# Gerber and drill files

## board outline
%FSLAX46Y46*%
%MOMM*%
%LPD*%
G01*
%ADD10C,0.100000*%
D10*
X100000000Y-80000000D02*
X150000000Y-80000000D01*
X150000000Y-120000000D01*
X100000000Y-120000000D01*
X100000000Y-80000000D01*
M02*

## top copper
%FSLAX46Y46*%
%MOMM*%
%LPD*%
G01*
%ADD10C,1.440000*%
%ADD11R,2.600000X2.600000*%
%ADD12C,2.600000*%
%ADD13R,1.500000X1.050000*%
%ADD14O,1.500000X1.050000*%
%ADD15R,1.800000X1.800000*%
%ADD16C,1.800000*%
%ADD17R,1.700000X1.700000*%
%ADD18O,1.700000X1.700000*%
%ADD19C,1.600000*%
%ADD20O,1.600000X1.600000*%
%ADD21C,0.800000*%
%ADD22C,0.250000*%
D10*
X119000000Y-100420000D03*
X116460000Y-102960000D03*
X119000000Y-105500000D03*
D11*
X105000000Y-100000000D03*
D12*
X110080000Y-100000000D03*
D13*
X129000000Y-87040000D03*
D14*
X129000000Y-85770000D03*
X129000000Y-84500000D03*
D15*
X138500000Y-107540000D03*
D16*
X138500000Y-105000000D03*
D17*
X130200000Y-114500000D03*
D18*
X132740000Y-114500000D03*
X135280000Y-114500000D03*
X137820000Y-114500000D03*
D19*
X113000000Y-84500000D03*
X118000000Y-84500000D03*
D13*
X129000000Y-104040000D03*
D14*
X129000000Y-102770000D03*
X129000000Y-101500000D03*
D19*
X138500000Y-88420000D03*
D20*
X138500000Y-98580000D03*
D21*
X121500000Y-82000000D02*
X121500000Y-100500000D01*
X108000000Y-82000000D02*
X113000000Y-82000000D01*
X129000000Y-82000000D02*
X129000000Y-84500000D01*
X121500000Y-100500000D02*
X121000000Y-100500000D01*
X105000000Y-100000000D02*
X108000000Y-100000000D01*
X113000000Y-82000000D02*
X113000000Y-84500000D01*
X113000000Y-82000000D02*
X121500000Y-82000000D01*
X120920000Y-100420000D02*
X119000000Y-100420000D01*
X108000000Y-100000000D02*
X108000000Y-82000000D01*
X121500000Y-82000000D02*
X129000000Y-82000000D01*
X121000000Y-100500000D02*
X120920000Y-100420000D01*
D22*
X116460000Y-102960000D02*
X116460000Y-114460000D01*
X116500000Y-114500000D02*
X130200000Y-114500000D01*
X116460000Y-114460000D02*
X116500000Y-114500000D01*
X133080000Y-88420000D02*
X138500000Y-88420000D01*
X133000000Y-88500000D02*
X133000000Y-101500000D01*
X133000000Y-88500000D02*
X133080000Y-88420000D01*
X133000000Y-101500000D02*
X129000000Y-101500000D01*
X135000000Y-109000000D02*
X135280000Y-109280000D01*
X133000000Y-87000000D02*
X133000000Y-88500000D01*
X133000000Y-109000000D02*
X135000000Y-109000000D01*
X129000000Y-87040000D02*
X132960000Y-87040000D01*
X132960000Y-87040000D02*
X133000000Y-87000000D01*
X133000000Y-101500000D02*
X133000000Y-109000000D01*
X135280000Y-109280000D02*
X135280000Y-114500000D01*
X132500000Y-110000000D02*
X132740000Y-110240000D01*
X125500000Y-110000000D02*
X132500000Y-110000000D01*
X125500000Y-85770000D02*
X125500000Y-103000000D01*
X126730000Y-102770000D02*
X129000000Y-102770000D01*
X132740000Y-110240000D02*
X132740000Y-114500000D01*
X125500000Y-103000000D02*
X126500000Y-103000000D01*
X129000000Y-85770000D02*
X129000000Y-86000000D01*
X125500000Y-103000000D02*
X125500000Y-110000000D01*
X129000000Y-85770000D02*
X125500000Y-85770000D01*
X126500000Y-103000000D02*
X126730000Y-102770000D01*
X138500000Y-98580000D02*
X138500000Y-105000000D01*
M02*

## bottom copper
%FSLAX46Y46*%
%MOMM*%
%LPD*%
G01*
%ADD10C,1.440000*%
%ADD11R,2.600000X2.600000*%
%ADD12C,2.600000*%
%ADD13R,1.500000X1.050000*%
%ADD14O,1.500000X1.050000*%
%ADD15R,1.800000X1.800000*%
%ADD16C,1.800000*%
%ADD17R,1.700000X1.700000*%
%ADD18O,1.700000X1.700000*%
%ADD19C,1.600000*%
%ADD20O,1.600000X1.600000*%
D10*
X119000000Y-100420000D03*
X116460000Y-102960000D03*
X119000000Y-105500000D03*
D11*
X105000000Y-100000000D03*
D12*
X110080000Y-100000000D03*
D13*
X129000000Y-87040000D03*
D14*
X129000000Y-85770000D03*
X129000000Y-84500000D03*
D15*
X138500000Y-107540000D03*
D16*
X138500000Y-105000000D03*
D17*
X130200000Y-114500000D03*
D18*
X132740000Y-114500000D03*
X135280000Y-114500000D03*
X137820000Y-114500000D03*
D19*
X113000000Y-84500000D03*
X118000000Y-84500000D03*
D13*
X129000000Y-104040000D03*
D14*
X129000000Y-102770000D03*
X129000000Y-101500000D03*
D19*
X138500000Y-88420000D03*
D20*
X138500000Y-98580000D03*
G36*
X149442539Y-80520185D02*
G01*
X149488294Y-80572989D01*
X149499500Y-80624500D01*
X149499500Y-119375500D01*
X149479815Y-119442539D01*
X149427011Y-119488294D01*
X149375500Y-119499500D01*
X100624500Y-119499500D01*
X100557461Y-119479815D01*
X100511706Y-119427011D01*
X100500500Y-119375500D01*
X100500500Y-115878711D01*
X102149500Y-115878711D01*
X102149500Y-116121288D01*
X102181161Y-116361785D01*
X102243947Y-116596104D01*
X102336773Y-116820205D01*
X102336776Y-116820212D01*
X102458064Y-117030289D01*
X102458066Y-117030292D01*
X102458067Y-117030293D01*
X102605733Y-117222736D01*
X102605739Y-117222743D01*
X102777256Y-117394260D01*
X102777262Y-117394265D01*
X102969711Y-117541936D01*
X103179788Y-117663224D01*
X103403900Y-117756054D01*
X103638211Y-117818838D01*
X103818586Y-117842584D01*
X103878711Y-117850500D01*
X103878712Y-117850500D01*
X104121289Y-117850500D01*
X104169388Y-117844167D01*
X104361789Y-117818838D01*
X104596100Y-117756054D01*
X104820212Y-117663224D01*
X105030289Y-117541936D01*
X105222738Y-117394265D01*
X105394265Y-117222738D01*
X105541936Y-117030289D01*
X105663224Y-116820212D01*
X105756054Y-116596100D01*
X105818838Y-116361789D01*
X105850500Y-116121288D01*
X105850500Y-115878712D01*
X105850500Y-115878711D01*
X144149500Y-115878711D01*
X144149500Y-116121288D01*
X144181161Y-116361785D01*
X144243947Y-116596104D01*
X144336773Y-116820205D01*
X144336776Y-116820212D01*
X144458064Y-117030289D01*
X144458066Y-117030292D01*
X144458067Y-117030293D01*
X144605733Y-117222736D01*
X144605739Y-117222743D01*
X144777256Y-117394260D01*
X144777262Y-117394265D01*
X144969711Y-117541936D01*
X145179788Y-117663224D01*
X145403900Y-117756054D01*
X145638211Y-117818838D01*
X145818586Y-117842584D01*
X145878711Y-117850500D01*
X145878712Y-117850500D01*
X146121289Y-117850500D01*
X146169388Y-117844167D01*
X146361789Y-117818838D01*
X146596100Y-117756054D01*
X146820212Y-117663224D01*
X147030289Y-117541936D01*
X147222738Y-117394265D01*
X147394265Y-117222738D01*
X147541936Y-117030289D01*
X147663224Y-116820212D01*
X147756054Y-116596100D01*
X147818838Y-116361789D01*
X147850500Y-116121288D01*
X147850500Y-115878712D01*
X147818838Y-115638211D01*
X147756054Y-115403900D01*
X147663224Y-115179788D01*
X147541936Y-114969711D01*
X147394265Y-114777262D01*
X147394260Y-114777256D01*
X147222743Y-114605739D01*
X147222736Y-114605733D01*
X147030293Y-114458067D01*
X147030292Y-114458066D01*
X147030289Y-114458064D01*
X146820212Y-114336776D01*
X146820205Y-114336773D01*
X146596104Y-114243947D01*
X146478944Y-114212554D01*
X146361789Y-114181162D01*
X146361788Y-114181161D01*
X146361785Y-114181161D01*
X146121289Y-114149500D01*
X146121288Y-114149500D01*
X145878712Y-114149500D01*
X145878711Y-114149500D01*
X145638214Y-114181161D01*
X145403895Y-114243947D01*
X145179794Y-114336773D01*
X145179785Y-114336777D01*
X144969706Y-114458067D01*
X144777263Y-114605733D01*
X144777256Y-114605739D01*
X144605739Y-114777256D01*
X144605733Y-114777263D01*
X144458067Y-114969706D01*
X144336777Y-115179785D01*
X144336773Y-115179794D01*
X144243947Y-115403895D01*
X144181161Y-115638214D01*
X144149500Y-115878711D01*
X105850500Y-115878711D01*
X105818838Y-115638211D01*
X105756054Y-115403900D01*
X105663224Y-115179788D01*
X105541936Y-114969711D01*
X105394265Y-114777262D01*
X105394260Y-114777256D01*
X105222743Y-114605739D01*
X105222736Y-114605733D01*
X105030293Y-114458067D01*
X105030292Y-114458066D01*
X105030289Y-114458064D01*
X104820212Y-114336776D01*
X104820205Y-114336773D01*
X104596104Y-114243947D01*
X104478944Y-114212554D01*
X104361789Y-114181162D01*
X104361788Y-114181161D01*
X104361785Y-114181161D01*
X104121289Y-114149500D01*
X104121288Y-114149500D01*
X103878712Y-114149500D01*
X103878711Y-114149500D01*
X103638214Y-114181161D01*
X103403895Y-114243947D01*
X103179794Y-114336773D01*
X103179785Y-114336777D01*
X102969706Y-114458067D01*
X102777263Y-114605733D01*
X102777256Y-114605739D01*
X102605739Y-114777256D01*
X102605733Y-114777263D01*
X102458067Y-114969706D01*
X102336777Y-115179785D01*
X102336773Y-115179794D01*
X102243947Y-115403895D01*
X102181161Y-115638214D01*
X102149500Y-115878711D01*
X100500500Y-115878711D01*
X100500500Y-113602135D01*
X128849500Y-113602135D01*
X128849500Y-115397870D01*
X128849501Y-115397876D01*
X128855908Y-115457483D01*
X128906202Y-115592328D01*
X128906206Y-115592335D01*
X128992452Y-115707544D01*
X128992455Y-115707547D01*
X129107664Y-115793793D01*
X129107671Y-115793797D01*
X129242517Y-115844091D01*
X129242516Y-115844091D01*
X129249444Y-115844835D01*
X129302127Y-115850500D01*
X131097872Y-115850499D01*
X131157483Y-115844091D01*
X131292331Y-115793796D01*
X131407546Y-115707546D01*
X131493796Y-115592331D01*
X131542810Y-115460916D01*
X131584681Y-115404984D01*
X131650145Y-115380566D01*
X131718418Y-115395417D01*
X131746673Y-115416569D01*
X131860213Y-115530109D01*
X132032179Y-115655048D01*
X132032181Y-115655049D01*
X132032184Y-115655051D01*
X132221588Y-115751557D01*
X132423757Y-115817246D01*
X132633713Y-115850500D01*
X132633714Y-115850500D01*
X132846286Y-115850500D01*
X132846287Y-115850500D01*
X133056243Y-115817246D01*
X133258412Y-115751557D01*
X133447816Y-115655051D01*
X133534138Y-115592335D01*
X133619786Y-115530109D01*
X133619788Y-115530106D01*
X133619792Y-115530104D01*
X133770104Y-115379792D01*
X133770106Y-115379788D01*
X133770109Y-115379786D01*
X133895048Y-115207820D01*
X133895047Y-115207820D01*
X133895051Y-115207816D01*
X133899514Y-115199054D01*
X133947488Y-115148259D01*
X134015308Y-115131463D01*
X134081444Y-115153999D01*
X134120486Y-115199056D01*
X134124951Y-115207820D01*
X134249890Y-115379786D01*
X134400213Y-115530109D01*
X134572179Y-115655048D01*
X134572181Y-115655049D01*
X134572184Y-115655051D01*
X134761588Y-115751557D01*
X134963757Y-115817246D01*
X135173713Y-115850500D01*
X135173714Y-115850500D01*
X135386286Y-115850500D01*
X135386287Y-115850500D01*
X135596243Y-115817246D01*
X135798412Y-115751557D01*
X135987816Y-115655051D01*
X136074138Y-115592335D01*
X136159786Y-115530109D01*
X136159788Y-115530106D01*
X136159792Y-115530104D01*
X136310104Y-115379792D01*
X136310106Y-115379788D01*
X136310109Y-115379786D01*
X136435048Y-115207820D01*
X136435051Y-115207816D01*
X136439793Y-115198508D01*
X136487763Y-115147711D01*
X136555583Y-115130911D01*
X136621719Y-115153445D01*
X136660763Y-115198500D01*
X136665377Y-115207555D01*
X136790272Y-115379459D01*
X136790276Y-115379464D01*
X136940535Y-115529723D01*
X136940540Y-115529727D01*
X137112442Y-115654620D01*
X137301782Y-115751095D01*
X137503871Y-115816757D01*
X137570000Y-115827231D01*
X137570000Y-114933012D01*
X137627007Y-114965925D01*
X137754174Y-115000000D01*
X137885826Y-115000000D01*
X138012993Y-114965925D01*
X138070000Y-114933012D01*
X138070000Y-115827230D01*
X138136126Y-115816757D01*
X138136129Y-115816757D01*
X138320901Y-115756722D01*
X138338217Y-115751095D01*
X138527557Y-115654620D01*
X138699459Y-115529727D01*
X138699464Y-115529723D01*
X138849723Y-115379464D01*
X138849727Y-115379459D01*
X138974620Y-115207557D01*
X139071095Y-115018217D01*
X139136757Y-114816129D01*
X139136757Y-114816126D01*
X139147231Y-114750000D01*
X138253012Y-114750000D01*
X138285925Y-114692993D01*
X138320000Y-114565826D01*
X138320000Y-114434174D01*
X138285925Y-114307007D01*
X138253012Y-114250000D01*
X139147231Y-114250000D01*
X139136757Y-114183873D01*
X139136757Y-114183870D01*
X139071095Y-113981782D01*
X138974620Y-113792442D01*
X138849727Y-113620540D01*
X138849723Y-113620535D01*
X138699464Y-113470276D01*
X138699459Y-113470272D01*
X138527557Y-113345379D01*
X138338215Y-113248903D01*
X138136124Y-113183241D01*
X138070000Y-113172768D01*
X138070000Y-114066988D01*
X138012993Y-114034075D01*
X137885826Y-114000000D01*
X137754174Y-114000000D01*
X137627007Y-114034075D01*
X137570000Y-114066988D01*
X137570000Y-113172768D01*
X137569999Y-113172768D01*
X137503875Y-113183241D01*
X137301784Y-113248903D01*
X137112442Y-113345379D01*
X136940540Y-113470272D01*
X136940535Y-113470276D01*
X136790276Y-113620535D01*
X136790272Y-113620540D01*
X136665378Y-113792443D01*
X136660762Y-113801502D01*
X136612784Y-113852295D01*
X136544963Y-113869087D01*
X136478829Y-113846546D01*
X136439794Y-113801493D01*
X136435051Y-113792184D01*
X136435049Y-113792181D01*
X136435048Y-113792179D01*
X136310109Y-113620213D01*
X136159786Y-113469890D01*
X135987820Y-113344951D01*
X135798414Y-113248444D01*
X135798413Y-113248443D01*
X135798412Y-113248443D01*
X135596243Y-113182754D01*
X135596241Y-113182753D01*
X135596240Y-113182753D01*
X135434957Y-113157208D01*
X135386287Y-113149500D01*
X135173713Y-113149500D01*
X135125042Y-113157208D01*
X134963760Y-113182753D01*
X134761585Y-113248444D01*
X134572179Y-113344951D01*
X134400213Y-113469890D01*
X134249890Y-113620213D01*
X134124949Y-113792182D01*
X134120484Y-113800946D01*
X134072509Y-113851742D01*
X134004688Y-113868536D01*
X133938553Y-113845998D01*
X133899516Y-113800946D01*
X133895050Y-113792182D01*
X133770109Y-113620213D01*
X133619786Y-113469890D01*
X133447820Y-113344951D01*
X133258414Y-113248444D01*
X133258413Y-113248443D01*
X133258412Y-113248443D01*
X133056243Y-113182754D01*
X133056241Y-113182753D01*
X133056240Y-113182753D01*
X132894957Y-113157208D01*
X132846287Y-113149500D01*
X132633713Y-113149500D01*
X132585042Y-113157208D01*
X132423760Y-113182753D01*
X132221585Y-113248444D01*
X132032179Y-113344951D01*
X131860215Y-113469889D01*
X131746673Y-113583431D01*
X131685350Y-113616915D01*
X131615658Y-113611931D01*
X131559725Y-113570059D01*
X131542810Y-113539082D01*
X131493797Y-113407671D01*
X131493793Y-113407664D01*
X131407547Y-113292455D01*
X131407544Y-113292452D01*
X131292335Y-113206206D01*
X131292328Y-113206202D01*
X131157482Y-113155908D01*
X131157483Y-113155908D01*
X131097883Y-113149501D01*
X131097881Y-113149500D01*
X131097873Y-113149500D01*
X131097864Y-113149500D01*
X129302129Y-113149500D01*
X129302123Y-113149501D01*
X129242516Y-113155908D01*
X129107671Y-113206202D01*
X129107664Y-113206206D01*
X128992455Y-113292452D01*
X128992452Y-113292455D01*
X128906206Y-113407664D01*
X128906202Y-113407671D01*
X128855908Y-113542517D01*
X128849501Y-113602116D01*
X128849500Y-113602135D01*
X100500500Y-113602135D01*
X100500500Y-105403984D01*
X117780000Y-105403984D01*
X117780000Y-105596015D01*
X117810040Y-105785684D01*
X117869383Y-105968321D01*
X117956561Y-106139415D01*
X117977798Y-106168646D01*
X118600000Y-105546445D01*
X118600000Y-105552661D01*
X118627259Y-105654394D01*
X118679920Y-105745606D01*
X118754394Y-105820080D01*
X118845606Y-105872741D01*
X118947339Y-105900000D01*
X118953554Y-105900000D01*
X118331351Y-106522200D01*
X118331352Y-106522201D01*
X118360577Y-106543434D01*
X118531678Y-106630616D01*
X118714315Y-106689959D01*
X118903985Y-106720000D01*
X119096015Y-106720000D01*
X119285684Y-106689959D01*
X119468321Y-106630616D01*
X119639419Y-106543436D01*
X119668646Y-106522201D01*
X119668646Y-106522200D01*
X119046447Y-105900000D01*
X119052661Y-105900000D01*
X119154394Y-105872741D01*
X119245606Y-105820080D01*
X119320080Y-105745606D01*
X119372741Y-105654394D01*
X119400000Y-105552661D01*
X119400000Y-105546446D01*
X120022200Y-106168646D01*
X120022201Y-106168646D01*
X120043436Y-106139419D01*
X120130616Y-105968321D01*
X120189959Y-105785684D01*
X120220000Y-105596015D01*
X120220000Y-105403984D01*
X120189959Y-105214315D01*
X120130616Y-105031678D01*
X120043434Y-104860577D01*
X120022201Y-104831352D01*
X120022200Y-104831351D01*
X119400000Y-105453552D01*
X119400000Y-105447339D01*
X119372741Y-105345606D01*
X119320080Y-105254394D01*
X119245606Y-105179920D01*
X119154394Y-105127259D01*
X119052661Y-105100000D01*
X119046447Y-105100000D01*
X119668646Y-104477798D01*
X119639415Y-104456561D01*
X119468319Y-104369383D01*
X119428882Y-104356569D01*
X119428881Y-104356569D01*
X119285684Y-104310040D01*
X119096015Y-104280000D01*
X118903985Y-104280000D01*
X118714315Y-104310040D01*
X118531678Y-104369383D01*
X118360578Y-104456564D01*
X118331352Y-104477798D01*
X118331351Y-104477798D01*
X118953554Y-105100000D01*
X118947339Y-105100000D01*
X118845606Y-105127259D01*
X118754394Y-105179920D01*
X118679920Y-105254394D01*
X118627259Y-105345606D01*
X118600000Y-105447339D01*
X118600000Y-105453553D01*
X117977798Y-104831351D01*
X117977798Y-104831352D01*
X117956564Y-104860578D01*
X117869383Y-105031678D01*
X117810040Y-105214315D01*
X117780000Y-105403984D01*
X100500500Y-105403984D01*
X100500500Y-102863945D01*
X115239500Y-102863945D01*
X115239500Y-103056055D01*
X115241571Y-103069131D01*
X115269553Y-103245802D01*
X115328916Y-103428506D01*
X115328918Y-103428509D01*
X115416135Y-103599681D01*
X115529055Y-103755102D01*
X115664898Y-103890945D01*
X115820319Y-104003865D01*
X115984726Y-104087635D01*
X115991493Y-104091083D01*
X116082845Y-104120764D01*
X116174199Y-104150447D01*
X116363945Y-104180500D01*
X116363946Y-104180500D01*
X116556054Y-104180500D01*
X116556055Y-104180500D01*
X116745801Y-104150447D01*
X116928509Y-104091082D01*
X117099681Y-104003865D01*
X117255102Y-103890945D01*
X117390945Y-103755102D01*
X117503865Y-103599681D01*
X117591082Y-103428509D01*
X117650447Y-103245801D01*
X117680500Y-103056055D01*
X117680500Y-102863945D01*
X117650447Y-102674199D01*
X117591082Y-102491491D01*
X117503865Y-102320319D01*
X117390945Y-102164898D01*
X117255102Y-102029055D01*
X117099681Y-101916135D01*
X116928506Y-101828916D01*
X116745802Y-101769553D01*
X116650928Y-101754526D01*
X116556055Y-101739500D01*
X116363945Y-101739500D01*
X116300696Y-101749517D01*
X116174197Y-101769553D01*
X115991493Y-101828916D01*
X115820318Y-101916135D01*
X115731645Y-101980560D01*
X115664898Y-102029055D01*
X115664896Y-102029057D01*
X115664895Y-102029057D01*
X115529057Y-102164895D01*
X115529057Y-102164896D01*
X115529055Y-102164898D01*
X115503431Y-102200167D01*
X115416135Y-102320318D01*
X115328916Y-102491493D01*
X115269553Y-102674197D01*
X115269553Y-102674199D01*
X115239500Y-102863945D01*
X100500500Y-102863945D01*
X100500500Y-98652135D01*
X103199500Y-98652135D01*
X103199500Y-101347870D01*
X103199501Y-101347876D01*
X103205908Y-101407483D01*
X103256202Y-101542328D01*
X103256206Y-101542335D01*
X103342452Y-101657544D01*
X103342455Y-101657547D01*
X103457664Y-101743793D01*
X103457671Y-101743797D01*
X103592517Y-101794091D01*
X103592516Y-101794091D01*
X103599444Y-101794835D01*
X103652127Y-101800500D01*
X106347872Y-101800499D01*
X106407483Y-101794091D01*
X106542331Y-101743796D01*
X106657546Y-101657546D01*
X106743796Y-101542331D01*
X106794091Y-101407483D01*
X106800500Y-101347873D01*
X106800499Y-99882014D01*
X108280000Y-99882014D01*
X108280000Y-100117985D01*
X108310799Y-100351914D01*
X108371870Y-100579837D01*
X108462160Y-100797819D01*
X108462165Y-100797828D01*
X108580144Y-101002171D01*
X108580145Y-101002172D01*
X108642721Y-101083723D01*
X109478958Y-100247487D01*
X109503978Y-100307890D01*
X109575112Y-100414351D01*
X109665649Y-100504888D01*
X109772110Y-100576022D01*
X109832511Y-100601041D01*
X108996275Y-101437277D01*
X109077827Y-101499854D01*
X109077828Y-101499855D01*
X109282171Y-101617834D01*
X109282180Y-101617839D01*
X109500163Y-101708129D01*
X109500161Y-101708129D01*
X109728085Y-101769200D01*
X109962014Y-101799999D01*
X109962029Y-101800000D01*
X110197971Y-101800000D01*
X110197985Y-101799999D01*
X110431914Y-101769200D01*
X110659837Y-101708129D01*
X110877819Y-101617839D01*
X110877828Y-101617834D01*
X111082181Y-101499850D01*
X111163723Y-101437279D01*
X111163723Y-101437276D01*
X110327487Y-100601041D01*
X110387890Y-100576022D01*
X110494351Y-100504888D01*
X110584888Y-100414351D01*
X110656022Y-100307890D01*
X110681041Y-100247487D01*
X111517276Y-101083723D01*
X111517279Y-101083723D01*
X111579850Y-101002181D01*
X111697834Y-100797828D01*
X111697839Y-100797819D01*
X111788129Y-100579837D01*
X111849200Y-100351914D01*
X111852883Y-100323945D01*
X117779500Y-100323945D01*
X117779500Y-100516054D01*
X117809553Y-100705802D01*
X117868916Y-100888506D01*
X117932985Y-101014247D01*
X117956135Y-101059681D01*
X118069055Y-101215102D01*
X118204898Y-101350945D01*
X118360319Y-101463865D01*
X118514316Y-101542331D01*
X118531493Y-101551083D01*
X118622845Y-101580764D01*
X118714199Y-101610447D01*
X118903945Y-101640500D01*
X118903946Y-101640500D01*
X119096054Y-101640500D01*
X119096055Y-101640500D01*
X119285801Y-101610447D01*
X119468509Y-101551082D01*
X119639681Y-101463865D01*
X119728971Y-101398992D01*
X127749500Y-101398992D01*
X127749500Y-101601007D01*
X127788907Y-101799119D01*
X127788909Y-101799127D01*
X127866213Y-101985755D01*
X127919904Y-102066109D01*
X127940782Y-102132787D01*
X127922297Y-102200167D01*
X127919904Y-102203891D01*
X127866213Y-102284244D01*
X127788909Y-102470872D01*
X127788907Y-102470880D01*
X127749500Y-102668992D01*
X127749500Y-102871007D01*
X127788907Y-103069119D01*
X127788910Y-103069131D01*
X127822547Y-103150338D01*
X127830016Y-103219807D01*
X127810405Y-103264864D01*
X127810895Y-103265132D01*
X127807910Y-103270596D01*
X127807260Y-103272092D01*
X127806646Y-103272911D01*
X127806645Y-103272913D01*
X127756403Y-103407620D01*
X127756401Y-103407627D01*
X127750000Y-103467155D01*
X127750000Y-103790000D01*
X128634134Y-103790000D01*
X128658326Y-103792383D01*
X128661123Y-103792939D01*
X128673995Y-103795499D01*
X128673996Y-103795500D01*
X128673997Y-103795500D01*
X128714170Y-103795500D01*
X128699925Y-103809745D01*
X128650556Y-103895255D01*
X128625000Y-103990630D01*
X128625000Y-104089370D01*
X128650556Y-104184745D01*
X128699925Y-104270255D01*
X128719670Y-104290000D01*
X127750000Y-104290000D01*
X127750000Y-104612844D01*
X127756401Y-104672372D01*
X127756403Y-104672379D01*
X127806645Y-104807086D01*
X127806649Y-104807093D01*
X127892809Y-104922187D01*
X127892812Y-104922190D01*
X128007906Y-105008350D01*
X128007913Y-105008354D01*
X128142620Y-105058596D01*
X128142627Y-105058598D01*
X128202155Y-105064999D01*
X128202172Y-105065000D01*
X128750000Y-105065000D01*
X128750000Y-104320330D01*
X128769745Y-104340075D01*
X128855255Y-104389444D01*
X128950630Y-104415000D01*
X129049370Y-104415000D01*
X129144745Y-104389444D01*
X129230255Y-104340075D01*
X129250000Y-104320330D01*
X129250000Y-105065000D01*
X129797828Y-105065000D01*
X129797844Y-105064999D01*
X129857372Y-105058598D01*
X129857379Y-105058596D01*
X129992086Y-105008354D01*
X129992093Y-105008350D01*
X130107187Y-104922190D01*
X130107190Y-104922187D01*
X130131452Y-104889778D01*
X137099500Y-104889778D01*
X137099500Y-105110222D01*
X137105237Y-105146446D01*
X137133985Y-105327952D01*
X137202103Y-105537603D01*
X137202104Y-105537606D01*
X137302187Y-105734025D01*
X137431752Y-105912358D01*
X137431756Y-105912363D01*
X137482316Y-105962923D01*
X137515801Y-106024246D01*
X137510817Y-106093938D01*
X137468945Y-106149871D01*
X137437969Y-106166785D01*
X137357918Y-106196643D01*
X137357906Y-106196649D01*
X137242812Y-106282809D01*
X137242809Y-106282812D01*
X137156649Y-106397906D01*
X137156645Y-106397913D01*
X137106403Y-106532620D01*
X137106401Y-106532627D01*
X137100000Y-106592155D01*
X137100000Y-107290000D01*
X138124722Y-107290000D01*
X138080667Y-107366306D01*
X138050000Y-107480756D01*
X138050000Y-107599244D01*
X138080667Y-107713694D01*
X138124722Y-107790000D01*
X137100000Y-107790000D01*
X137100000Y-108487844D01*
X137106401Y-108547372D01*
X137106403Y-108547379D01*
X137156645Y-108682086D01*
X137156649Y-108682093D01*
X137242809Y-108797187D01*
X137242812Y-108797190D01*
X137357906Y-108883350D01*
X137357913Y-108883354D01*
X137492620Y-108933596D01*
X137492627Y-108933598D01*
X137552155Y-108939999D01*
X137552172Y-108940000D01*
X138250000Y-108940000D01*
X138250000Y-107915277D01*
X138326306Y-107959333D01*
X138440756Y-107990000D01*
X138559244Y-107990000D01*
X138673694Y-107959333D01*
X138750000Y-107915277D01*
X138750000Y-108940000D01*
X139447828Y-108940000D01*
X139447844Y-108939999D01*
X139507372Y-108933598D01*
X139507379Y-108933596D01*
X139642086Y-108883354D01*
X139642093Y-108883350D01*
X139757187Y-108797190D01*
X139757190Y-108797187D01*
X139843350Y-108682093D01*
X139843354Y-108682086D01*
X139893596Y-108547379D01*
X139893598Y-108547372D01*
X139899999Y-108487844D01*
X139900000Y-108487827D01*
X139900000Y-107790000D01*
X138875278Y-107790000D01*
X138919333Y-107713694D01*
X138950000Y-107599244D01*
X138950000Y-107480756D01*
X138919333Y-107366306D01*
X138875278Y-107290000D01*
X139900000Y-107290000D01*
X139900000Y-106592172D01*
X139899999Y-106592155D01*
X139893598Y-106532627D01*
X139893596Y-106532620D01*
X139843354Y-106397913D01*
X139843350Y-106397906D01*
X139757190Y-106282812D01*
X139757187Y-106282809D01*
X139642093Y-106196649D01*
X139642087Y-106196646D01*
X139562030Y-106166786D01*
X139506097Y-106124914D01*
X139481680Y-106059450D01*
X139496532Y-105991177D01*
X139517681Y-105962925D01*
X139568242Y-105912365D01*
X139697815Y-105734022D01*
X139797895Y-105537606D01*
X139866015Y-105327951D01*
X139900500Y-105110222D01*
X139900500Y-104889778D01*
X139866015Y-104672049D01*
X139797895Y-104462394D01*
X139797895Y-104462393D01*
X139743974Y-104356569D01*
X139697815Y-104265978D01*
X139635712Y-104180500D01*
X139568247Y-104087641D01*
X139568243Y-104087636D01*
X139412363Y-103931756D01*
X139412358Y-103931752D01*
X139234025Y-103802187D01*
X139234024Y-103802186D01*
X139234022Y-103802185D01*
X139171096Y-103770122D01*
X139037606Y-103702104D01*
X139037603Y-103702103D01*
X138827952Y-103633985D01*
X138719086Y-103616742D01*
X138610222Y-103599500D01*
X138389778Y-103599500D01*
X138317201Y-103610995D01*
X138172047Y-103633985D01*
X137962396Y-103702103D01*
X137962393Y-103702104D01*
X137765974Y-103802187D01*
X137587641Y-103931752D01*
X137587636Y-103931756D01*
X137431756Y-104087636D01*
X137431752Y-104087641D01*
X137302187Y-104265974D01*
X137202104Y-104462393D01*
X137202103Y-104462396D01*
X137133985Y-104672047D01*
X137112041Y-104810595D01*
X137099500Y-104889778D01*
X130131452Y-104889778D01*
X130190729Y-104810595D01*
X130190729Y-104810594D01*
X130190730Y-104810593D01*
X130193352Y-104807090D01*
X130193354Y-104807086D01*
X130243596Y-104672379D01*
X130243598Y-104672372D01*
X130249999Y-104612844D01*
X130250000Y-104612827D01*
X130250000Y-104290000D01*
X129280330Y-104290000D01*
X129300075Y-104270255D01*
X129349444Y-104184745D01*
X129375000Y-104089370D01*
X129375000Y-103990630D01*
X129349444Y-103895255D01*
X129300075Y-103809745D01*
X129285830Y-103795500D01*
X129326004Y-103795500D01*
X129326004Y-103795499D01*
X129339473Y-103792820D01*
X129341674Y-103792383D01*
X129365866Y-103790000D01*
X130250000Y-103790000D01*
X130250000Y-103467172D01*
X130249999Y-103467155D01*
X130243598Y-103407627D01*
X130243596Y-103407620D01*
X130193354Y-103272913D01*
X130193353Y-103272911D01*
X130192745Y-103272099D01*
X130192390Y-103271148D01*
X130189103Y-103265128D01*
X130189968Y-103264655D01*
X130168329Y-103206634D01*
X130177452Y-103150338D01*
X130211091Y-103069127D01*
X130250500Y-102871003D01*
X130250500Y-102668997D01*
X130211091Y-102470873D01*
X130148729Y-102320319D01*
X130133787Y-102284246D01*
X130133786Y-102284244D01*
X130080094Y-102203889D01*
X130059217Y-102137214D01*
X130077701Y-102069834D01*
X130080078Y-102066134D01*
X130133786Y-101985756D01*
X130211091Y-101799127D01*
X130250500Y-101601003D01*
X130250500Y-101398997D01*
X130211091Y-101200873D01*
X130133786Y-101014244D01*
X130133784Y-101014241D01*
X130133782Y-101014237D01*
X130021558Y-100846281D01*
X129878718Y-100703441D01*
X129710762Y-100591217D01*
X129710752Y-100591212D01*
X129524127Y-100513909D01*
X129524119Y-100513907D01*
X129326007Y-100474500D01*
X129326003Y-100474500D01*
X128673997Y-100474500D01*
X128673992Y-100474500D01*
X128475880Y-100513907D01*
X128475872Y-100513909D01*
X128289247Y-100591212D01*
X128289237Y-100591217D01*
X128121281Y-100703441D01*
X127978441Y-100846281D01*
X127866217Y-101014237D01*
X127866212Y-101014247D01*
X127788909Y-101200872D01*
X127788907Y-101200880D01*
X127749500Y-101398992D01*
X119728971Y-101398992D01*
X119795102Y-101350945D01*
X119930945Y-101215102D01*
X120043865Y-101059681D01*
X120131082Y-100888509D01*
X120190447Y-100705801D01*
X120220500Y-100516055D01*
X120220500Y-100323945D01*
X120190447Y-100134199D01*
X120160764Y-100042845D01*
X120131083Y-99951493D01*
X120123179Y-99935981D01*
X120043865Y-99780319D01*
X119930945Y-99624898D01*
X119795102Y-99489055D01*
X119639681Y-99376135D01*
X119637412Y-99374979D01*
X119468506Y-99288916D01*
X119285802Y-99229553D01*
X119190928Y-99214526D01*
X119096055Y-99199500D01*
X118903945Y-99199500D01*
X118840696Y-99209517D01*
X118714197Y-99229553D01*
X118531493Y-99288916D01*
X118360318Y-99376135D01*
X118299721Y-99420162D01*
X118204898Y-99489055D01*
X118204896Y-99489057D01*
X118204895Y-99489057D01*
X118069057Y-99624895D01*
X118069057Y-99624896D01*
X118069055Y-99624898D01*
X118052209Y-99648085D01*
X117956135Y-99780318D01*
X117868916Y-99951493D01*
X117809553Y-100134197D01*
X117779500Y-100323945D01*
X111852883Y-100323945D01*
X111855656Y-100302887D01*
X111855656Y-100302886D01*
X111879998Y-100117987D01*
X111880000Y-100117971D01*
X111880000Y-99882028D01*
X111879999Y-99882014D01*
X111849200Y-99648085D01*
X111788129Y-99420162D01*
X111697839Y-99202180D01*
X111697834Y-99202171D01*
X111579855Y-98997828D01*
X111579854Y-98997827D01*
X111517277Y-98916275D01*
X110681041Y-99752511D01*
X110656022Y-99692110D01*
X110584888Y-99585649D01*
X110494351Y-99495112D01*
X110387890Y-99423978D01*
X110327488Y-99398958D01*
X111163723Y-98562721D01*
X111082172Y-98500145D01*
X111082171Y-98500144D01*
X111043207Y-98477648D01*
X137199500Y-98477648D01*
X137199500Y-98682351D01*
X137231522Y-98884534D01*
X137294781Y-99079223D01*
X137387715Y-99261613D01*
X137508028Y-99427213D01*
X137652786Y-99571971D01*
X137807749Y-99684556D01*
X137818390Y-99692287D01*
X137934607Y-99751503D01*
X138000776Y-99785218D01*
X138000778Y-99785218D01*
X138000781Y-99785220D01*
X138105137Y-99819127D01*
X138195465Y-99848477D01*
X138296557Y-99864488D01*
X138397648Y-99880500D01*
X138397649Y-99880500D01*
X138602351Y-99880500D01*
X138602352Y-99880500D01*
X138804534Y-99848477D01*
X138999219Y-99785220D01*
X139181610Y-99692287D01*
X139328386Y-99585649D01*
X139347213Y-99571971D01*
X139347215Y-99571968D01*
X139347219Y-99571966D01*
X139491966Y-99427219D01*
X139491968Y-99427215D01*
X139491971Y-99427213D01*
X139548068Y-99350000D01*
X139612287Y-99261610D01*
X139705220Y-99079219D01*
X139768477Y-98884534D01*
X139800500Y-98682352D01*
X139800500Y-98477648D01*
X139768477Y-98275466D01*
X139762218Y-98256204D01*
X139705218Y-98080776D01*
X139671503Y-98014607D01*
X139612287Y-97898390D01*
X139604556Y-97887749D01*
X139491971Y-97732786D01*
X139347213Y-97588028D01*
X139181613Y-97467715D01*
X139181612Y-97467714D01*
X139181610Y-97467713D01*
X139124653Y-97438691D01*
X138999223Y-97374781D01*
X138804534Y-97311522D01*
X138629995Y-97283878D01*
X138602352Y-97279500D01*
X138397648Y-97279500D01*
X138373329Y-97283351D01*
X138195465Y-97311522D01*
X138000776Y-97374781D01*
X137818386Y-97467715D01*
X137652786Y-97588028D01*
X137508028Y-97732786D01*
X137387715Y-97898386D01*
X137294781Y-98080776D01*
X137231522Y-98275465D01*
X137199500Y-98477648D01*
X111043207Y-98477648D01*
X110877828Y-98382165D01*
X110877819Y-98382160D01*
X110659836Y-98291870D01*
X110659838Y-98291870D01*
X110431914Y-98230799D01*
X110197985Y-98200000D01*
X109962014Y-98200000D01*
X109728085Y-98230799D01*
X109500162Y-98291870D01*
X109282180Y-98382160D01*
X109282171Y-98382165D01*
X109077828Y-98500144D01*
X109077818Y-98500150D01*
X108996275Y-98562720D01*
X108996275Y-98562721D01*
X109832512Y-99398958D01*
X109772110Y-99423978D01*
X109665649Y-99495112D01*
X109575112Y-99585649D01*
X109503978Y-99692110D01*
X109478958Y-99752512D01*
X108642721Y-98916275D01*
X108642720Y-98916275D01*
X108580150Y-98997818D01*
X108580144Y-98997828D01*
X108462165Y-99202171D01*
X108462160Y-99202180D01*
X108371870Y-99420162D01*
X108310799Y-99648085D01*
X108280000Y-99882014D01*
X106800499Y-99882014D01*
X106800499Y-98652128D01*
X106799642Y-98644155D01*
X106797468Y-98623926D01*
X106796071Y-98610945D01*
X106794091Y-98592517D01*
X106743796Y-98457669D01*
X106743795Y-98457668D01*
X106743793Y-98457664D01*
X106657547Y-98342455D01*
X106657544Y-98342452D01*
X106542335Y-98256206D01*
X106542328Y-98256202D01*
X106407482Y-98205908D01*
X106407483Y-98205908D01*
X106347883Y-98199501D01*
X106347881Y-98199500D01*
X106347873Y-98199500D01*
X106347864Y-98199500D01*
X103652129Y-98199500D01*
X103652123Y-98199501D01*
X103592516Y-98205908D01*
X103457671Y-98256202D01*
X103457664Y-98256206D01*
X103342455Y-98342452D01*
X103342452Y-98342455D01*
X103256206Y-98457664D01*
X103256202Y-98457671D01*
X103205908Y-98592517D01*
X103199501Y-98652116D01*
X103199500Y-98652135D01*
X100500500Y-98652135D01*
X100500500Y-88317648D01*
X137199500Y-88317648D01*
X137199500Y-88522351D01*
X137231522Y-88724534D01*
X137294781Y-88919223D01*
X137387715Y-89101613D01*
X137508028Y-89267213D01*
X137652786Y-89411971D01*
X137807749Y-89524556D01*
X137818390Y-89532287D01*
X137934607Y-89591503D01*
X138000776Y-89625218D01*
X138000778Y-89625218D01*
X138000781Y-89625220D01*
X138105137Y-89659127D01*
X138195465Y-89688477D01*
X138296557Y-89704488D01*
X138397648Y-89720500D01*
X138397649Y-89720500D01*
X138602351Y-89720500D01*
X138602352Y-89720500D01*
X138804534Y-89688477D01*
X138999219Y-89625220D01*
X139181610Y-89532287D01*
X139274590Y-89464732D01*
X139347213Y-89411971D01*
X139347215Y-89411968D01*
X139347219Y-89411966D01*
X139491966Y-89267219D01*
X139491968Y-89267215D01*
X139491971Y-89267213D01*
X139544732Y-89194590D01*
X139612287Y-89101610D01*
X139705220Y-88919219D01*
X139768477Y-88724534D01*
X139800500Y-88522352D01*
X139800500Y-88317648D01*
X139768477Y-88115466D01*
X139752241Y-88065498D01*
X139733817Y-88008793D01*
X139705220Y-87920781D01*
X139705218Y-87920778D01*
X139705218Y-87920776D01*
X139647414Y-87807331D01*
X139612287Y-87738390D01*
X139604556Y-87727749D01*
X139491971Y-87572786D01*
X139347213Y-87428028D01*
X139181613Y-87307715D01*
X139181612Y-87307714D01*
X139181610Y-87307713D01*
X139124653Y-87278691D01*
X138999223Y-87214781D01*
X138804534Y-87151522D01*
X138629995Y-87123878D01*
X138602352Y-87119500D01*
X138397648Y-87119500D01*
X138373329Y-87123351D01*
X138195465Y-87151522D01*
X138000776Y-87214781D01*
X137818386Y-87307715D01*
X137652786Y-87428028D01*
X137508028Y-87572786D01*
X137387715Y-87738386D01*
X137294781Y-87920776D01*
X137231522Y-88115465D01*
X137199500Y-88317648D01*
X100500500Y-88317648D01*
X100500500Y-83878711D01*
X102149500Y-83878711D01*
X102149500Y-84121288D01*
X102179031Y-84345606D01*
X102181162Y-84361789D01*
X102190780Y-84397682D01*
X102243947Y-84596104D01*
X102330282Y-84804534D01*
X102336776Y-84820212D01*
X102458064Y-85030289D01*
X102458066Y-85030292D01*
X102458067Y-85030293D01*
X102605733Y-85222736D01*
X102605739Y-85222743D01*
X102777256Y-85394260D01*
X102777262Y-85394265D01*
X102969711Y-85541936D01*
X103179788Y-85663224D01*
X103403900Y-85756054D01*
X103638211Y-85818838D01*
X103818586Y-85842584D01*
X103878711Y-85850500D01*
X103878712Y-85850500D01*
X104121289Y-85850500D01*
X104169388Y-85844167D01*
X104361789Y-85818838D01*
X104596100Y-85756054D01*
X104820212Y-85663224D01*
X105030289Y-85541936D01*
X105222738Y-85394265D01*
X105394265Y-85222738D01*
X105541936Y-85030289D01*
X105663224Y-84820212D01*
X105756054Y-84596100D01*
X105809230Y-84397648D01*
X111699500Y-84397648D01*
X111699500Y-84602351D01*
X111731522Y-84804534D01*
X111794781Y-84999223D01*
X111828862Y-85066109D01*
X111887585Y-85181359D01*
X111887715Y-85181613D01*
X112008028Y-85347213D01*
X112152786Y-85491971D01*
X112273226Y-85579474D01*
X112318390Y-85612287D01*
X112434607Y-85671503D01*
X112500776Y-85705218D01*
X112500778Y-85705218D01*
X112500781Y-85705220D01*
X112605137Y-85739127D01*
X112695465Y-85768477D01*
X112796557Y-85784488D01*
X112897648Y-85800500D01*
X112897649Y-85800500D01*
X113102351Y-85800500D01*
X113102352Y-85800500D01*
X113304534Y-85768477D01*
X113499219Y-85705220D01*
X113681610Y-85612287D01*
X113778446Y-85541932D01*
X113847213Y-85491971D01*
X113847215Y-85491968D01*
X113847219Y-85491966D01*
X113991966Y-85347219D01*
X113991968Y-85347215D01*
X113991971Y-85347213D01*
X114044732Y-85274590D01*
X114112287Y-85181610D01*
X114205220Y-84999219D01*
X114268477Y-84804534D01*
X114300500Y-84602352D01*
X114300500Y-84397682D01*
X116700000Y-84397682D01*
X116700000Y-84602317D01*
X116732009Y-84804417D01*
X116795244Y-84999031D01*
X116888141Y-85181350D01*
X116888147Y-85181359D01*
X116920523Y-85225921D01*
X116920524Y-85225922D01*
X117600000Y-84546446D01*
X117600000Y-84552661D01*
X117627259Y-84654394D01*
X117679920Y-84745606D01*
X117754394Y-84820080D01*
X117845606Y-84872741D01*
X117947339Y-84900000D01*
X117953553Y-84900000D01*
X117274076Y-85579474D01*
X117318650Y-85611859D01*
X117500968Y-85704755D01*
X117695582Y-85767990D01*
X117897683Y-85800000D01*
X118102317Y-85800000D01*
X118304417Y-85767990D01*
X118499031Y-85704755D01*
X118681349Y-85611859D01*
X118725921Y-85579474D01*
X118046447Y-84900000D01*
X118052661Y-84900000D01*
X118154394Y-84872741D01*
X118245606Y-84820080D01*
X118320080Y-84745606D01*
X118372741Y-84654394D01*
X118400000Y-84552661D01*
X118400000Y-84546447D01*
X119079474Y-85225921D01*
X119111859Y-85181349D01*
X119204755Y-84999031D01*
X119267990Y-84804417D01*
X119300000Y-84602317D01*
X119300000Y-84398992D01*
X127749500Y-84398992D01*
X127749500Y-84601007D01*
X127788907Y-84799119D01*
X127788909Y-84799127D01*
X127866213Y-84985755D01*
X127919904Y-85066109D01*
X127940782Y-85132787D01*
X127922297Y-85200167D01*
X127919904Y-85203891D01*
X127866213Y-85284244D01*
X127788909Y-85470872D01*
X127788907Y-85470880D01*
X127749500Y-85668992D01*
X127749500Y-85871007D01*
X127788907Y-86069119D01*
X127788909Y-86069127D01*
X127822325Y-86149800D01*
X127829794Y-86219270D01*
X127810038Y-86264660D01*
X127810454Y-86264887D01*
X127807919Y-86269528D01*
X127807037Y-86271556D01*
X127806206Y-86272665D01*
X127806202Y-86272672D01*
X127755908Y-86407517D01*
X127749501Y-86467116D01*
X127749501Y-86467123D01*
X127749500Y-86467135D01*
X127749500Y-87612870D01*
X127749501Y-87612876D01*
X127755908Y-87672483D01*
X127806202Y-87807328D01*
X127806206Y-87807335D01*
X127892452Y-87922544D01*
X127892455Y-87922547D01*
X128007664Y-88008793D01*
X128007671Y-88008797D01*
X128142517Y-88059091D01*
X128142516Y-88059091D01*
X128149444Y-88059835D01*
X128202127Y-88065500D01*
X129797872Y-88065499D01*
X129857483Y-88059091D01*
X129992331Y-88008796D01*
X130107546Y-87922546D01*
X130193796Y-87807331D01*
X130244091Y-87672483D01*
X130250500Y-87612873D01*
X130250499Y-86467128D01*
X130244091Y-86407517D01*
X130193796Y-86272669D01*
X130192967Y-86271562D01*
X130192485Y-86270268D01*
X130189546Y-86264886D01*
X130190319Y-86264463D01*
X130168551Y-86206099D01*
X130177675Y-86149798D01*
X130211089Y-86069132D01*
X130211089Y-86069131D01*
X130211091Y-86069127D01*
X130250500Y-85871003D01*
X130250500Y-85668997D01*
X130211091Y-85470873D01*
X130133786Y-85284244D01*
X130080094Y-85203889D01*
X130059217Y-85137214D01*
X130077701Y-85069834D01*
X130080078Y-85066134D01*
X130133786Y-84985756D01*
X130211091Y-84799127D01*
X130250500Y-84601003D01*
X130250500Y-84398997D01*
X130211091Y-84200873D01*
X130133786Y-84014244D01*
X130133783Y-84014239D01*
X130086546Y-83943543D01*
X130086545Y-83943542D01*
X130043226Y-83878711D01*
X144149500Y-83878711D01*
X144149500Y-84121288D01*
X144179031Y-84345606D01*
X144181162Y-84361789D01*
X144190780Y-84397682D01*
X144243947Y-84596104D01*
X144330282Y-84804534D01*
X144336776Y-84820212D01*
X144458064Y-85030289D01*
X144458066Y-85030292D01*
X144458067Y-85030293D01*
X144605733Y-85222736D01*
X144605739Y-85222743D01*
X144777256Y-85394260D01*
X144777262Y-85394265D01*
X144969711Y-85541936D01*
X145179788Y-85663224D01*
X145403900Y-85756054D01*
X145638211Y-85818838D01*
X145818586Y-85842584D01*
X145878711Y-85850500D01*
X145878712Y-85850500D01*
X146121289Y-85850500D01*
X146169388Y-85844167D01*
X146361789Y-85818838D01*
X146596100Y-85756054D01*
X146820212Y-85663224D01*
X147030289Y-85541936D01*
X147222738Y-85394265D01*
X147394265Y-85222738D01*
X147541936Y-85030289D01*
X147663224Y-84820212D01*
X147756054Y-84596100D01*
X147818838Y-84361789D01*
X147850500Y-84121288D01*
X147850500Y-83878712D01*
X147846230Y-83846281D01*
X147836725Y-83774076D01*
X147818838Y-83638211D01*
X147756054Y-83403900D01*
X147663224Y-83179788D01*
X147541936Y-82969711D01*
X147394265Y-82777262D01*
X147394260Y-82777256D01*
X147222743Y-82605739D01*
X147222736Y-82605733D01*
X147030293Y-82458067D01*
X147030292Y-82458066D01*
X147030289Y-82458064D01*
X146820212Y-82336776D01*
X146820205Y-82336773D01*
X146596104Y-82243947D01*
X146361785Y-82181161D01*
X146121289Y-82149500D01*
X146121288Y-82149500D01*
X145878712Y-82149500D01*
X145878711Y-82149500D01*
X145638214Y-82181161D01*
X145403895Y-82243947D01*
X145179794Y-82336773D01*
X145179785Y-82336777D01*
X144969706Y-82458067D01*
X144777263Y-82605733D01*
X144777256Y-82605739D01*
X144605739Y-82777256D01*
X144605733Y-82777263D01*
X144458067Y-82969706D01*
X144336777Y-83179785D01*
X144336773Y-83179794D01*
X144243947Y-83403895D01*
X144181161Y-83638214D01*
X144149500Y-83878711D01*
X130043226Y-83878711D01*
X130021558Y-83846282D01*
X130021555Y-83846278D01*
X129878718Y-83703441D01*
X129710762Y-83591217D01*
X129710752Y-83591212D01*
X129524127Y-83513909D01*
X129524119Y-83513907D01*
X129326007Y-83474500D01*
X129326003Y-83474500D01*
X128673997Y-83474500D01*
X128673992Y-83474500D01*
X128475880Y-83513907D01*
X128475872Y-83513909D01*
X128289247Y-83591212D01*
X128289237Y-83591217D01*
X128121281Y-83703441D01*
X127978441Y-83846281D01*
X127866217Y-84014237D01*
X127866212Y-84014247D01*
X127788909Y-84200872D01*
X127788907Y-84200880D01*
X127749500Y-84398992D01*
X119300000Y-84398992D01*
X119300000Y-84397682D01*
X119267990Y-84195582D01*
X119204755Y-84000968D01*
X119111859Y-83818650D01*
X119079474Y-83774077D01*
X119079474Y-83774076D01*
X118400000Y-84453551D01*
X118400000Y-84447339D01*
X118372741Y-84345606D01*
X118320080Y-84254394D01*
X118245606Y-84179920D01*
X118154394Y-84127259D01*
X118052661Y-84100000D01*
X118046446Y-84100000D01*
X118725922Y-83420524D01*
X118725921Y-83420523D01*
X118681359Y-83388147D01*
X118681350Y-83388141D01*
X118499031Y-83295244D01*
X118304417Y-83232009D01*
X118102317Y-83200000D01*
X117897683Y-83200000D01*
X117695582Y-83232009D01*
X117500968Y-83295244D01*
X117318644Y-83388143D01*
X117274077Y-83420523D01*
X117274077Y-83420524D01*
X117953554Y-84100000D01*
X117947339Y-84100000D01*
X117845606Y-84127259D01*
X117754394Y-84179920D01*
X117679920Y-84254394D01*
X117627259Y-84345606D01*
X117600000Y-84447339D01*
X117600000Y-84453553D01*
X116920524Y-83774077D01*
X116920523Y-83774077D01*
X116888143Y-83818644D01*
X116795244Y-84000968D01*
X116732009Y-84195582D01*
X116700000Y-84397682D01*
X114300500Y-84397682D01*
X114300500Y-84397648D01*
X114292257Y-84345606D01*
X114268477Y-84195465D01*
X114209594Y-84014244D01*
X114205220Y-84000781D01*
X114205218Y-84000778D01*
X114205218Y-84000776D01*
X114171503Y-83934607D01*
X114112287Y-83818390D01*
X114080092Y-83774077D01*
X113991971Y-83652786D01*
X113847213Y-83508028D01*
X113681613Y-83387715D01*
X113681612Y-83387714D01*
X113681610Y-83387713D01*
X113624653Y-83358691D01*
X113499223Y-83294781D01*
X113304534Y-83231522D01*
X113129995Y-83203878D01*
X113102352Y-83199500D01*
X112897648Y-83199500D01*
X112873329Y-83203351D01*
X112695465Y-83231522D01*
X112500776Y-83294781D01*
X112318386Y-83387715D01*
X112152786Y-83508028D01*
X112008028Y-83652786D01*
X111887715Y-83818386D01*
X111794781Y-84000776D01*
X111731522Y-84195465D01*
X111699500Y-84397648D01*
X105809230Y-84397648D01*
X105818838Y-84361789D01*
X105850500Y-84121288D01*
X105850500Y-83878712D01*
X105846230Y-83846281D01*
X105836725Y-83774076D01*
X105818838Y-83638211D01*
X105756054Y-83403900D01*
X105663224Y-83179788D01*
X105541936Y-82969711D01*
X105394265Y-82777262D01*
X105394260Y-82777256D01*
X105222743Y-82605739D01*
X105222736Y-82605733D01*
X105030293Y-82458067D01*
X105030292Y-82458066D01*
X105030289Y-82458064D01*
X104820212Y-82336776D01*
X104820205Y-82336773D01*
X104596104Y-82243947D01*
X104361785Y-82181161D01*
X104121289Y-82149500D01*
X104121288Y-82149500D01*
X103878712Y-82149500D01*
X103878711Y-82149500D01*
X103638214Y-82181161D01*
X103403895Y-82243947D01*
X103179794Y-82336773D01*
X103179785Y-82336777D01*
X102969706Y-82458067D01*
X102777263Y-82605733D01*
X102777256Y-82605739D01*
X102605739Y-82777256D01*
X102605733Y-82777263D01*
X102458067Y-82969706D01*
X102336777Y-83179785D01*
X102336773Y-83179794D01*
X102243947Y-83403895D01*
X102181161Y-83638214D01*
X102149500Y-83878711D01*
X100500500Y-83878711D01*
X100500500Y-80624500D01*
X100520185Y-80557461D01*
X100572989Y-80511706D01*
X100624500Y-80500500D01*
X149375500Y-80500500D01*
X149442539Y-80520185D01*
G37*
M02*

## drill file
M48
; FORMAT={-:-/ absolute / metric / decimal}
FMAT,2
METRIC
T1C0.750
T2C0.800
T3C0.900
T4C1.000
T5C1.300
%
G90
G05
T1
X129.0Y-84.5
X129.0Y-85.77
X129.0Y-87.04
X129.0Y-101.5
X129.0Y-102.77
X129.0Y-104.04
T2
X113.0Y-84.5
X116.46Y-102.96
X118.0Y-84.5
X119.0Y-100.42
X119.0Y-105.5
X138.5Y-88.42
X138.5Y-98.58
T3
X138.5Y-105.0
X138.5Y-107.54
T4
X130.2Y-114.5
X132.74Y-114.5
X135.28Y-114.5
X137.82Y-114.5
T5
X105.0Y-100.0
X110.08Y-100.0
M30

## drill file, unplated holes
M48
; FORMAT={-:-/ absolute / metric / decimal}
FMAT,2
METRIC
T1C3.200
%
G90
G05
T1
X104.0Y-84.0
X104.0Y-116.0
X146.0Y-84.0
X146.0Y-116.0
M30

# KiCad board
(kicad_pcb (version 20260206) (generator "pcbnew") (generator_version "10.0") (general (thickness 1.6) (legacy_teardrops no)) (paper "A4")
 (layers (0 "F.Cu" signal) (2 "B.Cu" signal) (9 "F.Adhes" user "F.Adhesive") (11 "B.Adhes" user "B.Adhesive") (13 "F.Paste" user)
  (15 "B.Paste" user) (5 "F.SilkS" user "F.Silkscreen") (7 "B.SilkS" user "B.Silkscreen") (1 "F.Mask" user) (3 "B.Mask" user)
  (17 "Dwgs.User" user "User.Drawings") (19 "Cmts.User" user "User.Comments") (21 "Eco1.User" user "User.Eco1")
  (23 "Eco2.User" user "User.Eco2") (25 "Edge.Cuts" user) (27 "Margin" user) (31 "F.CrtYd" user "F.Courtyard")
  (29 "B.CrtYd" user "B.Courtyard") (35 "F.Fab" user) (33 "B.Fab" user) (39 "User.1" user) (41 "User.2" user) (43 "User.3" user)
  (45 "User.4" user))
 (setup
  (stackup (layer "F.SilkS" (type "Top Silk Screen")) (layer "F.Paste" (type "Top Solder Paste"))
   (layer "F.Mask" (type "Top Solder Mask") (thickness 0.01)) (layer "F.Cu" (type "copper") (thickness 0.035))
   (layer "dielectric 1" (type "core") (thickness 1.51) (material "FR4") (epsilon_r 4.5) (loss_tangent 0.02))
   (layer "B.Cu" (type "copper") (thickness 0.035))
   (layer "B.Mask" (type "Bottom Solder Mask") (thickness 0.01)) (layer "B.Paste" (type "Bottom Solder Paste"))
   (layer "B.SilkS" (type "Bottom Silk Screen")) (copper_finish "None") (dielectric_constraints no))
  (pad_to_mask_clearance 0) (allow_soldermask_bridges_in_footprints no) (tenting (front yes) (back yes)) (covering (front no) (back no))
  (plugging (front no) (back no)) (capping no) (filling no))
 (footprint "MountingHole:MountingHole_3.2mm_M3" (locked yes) (layer "F.Cu") (at 146 84)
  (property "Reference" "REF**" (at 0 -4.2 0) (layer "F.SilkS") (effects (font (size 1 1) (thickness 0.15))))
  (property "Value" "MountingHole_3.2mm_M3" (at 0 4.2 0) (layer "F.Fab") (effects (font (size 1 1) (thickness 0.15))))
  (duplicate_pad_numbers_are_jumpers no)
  (pad "" np_thru_hole circle (at 0 0) (size 3.2 3.2) (drill 3.2) (layers "*.Cu" "*.Mask")))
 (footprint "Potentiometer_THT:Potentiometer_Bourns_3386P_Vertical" (layer "F.Cu") (at 119 100.42 180)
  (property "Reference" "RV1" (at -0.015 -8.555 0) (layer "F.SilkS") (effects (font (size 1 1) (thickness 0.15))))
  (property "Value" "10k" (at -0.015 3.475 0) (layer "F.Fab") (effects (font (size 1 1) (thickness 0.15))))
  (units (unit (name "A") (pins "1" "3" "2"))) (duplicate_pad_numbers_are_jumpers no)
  (pad "1" thru_hole circle (at 0 0 180) (size 1.44 1.44) (drill 0.8) (layers "*.Cu" "*.Mask") (remove_unused_layers no) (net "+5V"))
  (pad "2" thru_hole circle (at 2.54 -2.54 180) (size 1.44 1.44) (drill 0.8) (layers "*.Cu" "*.Mask") (remove_unused_layers no)
   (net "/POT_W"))
  (pad "3" thru_hole circle (at 0 -5.08 180) (size 1.44 1.44) (drill 0.8) (layers "*.Cu" "*.Mask") (remove_unused_layers no) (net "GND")))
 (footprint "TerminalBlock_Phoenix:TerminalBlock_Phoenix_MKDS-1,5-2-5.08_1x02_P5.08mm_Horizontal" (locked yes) (layer "F.Cu") (at 105 100)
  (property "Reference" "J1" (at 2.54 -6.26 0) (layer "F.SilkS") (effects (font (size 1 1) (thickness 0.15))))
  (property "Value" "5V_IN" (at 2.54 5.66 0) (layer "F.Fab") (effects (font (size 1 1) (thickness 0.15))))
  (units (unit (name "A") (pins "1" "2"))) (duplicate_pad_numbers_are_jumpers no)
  (pad "1" thru_hole rect (at 0 0) (size 2.6 2.6) (drill 1.3) (layers "*.Cu" "*.Mask") (remove_unused_layers no) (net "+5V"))
  (pad "2" thru_hole circle (at 5.08 0) (size 2.6 2.6) (drill 1.3) (layers "*.Cu" "*.Mask") (remove_unused_layers no) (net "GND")))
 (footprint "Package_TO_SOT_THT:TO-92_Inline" (layer "F.Cu") (at 129 87.04 90)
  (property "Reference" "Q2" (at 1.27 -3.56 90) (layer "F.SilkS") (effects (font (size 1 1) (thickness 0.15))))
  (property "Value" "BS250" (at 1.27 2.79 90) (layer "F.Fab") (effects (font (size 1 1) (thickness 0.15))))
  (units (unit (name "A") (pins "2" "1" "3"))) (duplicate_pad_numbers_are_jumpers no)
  (pad "1" thru_hole rect (at 0 0 90) (size 1.05 1.5) (drill 0.75) (layers "*.Cu" "*.Mask") (remove_unused_layers no) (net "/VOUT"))
  (pad "2" thru_hole oval (at 1.27 0 90) (size 1.05 1.5) (drill 0.75) (layers "*.Cu" "*.Mask") (remove_unused_layers no) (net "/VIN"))
  (pad "3" thru_hole oval (at 2.54 0 90) (size 1.05 1.5) (drill 0.75) (layers "*.Cu" "*.Mask") (remove_unused_layers no) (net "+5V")))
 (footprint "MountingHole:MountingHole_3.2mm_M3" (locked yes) (layer "F.Cu") (at 104 84)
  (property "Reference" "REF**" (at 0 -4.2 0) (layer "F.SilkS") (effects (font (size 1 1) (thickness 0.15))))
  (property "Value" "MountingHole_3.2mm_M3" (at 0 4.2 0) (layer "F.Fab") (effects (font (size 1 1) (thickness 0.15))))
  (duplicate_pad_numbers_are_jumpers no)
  (pad "" np_thru_hole circle (at 0 0) (size 3.2 3.2) (drill 3.2) (layers "*.Cu" "*.Mask")))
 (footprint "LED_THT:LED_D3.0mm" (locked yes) (layer "F.Cu") (at 138.5 107.54 90)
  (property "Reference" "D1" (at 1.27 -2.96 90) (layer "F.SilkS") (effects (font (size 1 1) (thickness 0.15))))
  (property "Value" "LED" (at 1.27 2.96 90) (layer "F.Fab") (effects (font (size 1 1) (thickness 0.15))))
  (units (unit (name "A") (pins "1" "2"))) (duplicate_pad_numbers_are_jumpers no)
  (pad "1" thru_hole rect (at 0 0 90) (size 1.8 1.8) (drill 0.9) (layers "*.Cu" "*.Mask") (remove_unused_layers no) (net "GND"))
  (pad "2" thru_hole circle (at 2.54 0 90) (size 1.8 1.8) (drill 0.9) (layers "*.Cu" "*.Mask") (remove_unused_layers no) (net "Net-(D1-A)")))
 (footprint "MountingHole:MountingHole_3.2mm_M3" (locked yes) (layer "F.Cu") (at 104 116)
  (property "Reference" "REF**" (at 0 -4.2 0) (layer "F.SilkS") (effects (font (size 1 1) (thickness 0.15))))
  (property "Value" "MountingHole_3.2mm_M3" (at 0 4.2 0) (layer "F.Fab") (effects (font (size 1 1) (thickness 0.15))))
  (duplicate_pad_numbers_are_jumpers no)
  (pad "" np_thru_hole circle (at 0 0) (size 3.2 3.2) (drill 3.2) (layers "*.Cu" "*.Mask")))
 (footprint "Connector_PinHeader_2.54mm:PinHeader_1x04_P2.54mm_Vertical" (layer "F.Cu") (at 130.2 114.5 90)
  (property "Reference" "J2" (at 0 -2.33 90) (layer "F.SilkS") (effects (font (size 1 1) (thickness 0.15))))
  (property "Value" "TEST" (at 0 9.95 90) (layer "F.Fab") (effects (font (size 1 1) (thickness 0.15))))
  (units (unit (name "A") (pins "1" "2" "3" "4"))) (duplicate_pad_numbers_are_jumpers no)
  (pad "1" thru_hole rect (at 0 0 90) (size 1.7 1.7) (drill 1) (layers "*.Cu" "*.Mask") (remove_unused_layers no) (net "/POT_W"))
  (pad "2" thru_hole oval (at 0 2.54 90) (size 1.7 1.7) (drill 1) (layers "*.Cu" "*.Mask") (remove_unused_layers no) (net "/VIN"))
  (pad "3" thru_hole oval (at 0 5.08 90) (size 1.7 1.7) (drill 1) (layers "*.Cu" "*.Mask") (remove_unused_layers no) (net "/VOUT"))
  (pad "4" thru_hole oval (at 0 7.62 90) (size 1.7 1.7) (drill 1) (layers "*.Cu" "*.Mask") (remove_unused_layers no) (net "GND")))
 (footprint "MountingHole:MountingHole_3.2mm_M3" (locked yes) (layer "F.Cu") (at 146 116)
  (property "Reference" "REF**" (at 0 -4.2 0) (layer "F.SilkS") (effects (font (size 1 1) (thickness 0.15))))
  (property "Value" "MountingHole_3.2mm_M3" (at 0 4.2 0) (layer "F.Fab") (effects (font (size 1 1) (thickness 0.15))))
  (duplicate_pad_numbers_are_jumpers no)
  (pad "" np_thru_hole circle (at 0 0) (size 3.2 3.2) (drill 3.2) (layers "*.Cu" "*.Mask")))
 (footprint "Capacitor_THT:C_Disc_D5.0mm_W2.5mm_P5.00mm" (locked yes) (layer "F.Cu") (at 113 84.5)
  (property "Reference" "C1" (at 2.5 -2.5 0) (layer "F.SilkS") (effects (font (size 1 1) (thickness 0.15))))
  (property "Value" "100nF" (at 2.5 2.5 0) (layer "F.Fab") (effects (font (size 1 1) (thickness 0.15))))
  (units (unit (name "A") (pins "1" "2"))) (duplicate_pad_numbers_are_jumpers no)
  (pad "1" thru_hole circle (at 0 0) (size 1.6 1.6) (drill 0.8) (layers "*.Cu" "*.Mask") (remove_unused_layers no) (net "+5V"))
  (pad "2" thru_hole circle (at 5 0) (size 1.6 1.6) (drill 0.8) (layers "*.Cu" "*.Mask") (remove_unused_layers no) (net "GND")))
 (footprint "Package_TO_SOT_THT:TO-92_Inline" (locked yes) (layer "F.Cu") (at 129 104.04 90)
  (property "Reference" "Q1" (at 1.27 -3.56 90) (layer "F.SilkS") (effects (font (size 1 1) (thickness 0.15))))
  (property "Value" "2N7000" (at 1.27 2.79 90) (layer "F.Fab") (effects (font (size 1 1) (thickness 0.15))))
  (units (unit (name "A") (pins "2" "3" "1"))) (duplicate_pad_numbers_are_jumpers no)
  (pad "1" thru_hole rect (at 0 0 90) (size 1.05 1.5) (drill 0.75) (layers "*.Cu" "*.Mask") (remove_unused_layers no) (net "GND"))
  (pad "2" thru_hole oval (at 1.27 0 90) (size 1.05 1.5) (drill 0.75) (layers "*.Cu" "*.Mask") (remove_unused_layers no) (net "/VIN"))
  (pad "3" thru_hole oval (at 2.54 0 90) (size 1.05 1.5) (drill 0.75) (layers "*.Cu" "*.Mask") (remove_unused_layers no) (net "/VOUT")))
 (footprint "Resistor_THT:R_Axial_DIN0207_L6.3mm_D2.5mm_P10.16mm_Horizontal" (layer "F.Cu") (at 138.5 88.42 -90)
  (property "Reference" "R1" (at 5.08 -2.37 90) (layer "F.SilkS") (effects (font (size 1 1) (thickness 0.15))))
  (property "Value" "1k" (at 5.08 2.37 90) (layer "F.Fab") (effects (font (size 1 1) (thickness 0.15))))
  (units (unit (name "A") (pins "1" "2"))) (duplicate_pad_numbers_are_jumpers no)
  (pad "1" thru_hole circle (at 0 0 270) (size 1.6 1.6) (drill 0.8) (layers "*.Cu" "*.Mask") (remove_unused_layers no) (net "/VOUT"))
  (pad "2" thru_hole oval (at 10.16 0 270) (size 1.6 1.6) (drill 0.8) (layers "*.Cu" "*.Mask") (remove_unused_layers no) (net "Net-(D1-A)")))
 (gr_rect (start 100 80) (end 150 120) (stroke (width 0.1) (type solid)) (fill no) (layer "Edge.Cuts"))
 (segment (start 121.5 82) (end 121.5 100.5) (width 0.8) (layer "F.Cu") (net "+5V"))
 (segment (start 108 82) (end 113 82) (width 0.8) (layer "F.Cu") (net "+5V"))
 (segment (start 129 82) (end 129 84.5) (width 0.8) (layer "F.Cu") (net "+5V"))
 (segment (start 121.5 100.5) (end 121 100.5) (width 0.8) (layer "F.Cu") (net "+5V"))
 (segment (start 105 100) (end 108 100) (width 0.8) (layer "F.Cu") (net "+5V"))
 (segment (start 113 82) (end 113 84.5) (width 0.8) (layer "F.Cu") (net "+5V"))
 (segment (start 113 82) (end 121.5 82) (width 0.8) (layer "F.Cu") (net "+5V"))
 (segment (start 120.92 100.42) (end 119 100.42) (width 0.8) (layer "F.Cu") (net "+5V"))
 (segment (start 108 100) (end 108 82) (width 0.8) (layer "F.Cu") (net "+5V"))
 (segment (start 121.5 82) (end 129 82) (width 0.8) (layer "F.Cu") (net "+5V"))
 (segment (start 121 100.5) (end 120.92 100.42) (width 0.8) (layer "F.Cu") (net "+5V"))
 (segment (start 116.46 102.96) (end 116.46 114.46) (width 0.25) (layer "F.Cu") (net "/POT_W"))
 (segment (start 116.5 114.5) (end 130.2 114.5) (width 0.25) (layer "F.Cu") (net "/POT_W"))
 (segment (start 116.46 114.46) (end 116.5 114.5) (width 0.25) (layer "F.Cu") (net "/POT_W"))
 (segment (start 133.08 88.42) (end 138.5 88.42) (width 0.25) (layer "F.Cu") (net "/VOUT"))
 (segment (start 133 88.5) (end 133 101.5) (width 0.25) (layer "F.Cu") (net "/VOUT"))
 (segment (start 133 88.5) (end 133.08 88.42) (width 0.25) (layer "F.Cu") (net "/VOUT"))
 (segment (start 133 101.5) (end 129 101.5) (width 0.25) (layer "F.Cu") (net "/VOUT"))
 (segment (start 135 109) (end 135.28 109.28) (width 0.25) (layer "F.Cu") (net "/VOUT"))
 (segment (start 133 87) (end 133 88.5) (width 0.25) (layer "F.Cu") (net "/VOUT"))
 (segment (start 133 109) (end 135 109) (width 0.25) (layer "F.Cu") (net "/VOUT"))
 (segment (start 129 87.04) (end 132.96 87.04) (width 0.25) (layer "F.Cu") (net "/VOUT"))
 (segment (start 132.96 87.04) (end 133 87) (width 0.25) (layer "F.Cu") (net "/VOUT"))
 (segment (start 133 101.5) (end 133 109) (width 0.25) (layer "F.Cu") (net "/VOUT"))
 (segment (start 135.28 109.28) (end 135.28 114.5) (width 0.25) (layer "F.Cu") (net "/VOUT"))
 (segment (start 132.5 110) (end 132.74 110.24) (width 0.25) (layer "F.Cu") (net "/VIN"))
 (segment (start 125.5 110) (end 132.5 110) (width 0.25) (layer "F.Cu") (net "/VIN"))
 (segment (start 125.5 85.77) (end 125.5 103) (width 0.25) (layer "F.Cu") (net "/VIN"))
 (segment (start 126.73 102.77) (end 129 102.77) (width 0.25) (layer "F.Cu") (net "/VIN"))
 (segment (start 132.74 110.24) (end 132.74 114.5) (width 0.25) (layer "F.Cu") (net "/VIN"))
 (segment (start 125.5 103) (end 126.5 103) (width 0.25) (layer "F.Cu") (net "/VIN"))
 (segment (start 129 85.77) (end 129 86) (width 0.25) (layer "F.Cu") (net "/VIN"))
 (segment (start 125.5 103) (end 125.5 110) (width 0.25) (layer "F.Cu") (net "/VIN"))
 (segment (start 129 85.77) (end 125.5 85.77) (width 0.25) (layer "F.Cu") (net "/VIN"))
 (segment (start 126.5 103) (end 126.73 102.77) (width 0.25) (layer "F.Cu") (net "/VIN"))
 (segment (start 138.5 98.58) (end 138.5 105) (width 0.25) (layer "F.Cu") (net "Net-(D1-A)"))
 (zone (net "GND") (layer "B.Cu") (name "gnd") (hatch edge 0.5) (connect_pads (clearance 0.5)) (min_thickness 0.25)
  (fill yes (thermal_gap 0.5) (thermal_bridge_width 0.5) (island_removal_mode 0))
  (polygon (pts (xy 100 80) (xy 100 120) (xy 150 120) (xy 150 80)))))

